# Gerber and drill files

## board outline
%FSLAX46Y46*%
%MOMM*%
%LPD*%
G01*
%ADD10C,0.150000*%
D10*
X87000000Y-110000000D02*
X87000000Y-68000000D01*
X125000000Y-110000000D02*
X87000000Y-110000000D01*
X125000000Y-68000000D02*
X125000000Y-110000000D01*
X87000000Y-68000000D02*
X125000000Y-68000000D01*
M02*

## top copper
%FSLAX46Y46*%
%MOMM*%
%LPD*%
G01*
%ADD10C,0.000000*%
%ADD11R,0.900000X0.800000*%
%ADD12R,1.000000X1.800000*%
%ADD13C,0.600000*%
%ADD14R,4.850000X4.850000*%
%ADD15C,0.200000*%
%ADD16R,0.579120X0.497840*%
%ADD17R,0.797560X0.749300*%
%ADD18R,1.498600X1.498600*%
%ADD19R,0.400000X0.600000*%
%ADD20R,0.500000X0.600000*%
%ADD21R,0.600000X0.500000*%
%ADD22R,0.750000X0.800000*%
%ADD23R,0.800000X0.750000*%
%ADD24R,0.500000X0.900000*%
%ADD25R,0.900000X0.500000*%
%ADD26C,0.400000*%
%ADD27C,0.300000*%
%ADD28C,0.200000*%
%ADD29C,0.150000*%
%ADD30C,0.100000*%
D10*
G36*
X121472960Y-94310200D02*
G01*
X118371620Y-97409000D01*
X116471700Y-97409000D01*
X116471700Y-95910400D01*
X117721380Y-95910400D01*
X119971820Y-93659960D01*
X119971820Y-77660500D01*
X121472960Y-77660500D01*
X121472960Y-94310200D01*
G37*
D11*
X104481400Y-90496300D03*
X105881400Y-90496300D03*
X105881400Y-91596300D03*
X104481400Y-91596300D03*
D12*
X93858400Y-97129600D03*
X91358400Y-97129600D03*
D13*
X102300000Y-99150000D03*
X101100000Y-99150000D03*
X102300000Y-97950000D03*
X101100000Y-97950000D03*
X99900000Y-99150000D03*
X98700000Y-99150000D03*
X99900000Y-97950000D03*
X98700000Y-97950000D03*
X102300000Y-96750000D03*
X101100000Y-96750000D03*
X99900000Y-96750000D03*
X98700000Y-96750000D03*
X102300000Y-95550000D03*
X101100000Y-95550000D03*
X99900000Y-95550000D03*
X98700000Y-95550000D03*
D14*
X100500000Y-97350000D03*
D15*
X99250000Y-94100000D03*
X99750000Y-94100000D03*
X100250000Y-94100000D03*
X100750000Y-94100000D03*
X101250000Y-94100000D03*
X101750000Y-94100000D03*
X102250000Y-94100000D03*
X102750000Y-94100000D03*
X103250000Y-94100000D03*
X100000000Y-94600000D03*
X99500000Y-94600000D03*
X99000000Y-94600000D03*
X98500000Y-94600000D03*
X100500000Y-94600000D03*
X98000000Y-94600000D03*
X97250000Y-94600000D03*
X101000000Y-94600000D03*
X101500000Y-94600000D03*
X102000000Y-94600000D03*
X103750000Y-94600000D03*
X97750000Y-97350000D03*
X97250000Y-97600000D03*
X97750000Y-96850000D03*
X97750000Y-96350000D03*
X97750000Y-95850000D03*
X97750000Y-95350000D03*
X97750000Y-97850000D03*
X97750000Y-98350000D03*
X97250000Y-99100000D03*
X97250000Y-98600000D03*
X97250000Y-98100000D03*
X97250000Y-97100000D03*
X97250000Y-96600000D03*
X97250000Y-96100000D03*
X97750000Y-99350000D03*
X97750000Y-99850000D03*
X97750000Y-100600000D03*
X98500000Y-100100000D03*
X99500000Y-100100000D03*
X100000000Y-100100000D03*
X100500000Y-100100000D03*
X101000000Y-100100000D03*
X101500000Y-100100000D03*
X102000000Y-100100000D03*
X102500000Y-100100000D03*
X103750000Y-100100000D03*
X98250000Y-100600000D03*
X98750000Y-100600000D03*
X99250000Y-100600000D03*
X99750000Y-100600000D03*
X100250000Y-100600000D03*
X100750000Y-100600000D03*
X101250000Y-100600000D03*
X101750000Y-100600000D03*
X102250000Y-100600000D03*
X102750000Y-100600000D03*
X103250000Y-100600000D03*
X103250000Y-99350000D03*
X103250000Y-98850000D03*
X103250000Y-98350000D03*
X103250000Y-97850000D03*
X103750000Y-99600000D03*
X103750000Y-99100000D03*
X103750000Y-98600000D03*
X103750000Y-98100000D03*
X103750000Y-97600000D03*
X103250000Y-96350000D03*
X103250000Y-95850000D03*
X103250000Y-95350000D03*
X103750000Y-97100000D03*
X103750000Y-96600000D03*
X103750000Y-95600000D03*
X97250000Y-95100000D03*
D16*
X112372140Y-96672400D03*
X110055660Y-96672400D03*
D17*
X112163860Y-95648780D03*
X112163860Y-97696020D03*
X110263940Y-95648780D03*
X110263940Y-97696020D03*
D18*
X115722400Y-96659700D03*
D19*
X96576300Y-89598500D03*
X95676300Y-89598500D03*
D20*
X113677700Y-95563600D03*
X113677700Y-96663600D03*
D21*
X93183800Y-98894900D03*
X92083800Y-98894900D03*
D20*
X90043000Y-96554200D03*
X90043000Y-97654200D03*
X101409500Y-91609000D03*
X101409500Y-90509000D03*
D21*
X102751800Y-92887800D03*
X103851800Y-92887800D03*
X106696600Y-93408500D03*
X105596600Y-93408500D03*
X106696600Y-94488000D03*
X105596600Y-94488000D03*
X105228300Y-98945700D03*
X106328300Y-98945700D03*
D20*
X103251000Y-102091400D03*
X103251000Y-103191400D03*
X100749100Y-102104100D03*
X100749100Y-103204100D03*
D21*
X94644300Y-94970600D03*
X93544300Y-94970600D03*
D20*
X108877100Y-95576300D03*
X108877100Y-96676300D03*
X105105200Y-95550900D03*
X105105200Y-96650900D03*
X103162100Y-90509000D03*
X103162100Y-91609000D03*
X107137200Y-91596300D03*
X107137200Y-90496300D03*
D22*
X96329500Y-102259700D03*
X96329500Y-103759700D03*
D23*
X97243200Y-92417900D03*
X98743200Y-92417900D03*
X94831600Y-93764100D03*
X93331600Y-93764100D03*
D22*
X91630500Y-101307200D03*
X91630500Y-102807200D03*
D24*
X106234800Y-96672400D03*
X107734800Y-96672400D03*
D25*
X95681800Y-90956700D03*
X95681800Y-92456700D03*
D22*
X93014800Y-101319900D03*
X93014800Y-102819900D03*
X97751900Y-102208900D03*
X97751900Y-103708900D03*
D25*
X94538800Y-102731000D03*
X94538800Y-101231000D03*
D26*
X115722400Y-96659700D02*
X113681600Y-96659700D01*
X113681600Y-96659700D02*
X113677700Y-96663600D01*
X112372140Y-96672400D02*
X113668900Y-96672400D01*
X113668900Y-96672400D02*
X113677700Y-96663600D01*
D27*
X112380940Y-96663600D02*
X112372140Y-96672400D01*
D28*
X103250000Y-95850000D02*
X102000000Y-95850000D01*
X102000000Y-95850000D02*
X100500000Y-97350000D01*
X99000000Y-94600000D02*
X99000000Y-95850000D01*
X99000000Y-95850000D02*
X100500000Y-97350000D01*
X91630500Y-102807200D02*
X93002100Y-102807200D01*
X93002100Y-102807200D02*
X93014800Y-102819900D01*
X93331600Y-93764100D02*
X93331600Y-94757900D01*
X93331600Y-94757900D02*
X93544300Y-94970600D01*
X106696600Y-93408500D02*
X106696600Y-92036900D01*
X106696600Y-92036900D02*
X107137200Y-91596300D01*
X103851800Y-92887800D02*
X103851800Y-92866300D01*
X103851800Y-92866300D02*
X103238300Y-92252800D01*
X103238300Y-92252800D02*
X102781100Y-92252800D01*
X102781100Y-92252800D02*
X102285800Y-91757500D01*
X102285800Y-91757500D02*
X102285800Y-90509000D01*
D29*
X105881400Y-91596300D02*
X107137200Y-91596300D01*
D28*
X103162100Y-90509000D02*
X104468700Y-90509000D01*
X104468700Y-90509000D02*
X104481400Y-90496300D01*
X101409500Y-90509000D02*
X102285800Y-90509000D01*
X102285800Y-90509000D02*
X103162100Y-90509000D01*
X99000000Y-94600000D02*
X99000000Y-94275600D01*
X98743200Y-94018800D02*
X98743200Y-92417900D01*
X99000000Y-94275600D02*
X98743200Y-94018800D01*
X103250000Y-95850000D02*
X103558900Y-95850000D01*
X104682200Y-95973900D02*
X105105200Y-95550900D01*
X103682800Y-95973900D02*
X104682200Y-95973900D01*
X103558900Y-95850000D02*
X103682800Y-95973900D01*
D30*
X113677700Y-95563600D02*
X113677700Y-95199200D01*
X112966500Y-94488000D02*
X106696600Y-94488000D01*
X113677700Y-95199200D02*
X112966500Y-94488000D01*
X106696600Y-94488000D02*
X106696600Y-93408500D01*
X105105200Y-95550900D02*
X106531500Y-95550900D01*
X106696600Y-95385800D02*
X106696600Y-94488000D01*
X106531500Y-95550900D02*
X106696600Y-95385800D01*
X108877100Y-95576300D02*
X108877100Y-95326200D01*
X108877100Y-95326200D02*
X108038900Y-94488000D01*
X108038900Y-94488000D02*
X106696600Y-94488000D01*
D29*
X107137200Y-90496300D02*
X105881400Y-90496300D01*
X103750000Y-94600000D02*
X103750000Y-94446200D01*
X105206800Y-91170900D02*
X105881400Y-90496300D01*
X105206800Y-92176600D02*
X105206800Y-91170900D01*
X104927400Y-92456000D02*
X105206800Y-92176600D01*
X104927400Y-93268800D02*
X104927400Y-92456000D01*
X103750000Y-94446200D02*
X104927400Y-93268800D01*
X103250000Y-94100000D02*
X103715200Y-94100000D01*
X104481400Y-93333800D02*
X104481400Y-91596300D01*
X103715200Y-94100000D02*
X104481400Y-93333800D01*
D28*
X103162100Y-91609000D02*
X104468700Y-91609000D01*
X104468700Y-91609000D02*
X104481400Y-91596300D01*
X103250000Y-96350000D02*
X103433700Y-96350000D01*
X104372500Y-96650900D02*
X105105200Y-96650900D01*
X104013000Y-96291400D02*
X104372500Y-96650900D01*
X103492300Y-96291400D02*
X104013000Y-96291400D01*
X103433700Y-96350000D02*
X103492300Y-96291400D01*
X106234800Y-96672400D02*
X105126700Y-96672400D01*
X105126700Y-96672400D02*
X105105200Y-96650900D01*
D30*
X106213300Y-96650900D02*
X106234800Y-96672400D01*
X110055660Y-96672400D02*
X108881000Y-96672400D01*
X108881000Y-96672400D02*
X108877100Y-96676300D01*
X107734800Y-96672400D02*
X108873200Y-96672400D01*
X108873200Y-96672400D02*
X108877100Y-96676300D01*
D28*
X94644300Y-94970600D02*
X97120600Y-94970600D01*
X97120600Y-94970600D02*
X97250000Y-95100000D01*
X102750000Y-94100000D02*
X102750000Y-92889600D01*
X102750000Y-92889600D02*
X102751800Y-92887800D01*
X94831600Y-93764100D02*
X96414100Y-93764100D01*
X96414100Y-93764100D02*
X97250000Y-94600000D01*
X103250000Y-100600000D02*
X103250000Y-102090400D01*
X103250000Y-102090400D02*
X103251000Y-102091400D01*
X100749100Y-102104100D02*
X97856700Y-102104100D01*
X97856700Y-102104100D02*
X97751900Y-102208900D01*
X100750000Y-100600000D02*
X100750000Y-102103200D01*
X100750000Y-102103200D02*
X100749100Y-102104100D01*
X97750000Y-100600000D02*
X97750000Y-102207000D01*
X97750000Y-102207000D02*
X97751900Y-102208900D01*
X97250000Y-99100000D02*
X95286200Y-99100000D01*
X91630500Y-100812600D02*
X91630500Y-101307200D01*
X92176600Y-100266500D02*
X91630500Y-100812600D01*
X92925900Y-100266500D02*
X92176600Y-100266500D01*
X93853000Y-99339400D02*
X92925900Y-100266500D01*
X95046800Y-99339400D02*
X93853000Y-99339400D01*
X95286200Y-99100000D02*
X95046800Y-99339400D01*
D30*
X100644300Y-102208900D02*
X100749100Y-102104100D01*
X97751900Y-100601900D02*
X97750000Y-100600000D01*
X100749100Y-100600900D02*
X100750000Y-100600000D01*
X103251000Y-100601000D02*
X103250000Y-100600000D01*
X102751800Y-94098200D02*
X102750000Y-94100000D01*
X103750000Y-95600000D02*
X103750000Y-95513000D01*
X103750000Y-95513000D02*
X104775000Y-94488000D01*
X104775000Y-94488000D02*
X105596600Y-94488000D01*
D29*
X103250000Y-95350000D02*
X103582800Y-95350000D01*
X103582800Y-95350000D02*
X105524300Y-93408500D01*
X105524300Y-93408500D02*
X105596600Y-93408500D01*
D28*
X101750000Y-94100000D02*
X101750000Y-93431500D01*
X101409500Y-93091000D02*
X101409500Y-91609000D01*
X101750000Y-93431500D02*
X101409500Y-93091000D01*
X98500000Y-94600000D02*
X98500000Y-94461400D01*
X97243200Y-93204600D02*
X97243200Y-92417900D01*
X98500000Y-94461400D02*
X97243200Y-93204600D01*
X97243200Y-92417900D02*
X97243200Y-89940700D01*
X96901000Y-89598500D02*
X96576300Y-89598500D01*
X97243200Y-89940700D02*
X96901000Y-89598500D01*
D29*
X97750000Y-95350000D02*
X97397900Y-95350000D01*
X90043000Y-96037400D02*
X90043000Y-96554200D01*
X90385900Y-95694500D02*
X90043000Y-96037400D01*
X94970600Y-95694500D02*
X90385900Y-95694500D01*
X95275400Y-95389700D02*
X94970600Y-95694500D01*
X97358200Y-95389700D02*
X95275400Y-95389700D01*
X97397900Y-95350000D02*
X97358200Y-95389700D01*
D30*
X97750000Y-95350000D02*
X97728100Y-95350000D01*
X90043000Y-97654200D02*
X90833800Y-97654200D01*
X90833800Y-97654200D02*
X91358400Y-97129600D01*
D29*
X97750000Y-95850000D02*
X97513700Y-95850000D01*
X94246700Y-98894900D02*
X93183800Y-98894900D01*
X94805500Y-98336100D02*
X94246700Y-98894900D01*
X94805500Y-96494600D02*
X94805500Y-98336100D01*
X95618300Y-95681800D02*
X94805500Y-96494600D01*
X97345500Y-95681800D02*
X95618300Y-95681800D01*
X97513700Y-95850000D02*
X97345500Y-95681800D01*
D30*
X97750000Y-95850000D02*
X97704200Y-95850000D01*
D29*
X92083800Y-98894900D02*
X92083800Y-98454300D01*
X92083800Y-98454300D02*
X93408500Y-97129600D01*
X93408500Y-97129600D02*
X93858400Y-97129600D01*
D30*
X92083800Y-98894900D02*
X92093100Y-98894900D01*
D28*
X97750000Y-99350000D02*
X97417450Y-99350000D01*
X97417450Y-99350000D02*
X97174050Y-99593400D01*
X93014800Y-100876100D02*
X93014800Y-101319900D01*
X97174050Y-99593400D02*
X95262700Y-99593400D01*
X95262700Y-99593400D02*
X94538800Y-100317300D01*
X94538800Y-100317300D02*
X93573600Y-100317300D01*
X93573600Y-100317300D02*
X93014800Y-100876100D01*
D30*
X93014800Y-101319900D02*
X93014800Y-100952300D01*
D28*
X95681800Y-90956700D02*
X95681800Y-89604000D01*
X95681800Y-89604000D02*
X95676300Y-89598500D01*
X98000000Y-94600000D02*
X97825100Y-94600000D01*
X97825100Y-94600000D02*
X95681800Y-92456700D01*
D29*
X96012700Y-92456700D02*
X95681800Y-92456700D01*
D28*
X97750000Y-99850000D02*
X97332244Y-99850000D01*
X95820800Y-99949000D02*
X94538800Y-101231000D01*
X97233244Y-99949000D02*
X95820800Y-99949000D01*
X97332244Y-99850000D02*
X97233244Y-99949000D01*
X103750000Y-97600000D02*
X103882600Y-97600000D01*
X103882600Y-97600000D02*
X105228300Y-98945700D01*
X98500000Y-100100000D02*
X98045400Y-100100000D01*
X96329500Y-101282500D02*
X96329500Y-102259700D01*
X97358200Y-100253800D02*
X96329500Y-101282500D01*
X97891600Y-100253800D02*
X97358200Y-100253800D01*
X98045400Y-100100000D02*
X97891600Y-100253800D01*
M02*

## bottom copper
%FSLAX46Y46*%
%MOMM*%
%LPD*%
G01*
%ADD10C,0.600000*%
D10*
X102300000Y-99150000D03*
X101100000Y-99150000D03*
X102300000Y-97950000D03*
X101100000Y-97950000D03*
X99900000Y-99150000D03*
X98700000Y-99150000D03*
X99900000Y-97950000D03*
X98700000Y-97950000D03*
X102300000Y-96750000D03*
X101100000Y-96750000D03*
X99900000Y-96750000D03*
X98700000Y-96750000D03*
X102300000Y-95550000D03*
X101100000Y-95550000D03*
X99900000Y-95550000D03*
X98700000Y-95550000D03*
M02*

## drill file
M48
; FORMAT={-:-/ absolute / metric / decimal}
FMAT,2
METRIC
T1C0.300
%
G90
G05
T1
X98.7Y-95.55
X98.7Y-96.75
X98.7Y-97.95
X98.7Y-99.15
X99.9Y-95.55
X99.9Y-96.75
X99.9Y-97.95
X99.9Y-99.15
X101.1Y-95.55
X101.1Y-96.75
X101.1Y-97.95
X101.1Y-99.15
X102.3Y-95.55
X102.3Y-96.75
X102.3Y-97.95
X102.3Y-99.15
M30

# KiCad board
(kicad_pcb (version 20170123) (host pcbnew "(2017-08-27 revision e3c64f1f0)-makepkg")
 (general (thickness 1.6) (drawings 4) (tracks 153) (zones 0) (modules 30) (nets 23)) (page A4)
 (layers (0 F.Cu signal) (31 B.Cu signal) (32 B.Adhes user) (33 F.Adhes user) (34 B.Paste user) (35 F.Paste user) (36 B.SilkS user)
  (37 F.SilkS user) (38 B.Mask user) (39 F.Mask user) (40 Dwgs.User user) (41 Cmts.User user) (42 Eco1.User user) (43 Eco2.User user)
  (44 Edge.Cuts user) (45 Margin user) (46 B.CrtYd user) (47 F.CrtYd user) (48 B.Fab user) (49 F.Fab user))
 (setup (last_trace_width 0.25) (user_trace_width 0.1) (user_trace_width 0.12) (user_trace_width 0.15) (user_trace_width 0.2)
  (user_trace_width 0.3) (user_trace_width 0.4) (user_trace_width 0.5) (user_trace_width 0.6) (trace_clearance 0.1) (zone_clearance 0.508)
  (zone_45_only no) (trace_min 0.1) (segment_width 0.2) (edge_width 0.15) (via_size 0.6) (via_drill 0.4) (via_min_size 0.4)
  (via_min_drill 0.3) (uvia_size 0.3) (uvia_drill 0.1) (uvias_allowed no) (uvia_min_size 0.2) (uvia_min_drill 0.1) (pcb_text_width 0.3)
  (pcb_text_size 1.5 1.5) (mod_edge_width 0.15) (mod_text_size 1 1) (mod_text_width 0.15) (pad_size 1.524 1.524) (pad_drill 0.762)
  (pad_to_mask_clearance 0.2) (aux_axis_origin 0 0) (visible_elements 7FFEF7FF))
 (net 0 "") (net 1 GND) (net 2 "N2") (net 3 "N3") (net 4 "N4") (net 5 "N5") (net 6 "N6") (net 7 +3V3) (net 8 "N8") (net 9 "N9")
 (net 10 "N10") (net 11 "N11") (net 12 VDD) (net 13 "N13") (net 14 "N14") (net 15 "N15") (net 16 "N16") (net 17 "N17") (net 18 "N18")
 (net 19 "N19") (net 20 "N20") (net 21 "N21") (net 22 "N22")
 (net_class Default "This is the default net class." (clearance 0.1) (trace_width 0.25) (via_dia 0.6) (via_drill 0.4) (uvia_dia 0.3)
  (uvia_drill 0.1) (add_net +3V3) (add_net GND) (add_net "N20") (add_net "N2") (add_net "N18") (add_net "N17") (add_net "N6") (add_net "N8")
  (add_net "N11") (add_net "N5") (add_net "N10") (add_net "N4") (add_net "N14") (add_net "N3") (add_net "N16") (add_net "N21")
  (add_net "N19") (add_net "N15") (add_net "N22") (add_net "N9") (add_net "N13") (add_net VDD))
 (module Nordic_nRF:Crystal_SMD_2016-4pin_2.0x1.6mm (layer F.Cu) (at 105.1814 91.0463)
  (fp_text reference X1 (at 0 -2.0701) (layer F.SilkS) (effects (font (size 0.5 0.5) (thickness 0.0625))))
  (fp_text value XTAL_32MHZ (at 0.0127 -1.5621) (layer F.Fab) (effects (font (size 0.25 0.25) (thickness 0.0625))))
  (pad 4 smd rect (at -0.7 -0.55) (size 0.9 0.8) (layers F.Cu F.Paste F.Mask) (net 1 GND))
  (pad 3 smd rect (at 0.7 -0.55) (size 0.9 0.8) (layers F.Cu F.Paste F.Mask) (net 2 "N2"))
  (pad 2 smd rect (at 0.7 0.55) (size 0.9 0.8) (layers F.Cu F.Paste F.Mask) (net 1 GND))
  (pad 1 smd rect (at -0.7 0.55) (size 0.9 0.8) (layers F.Cu F.Paste F.Mask) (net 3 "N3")))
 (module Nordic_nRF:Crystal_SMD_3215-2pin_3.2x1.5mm (layer F.Cu) (at 92.6084 97.1296 180)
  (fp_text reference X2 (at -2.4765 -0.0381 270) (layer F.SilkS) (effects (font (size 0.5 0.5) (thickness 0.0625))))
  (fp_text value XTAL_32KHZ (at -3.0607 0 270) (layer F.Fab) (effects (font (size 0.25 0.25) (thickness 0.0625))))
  (pad 2 smd rect (at -1.25 0 180) (size 1 1.8) (layers F.Cu F.Paste F.Mask) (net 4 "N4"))
  (pad 1 smd rect (at 1.25 0 180) (size 1 1.8) (layers F.Cu F.Paste F.Mask) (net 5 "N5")))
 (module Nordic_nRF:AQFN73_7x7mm (layer F.Cu) (at 100.5 97.35)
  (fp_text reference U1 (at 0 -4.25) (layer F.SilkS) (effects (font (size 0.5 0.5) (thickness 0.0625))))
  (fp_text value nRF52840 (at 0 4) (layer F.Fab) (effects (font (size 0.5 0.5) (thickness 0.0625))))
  (pad 74 thru_hole circle (at 1.8 1.8) (size 0.6 0.6) (drill 0.3) (layers *.Cu B.Mask) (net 1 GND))
  (pad 74 thru_hole circle (at 0.6 1.8) (size 0.6 0.6) (drill 0.3) (layers *.Cu B.Mask) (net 1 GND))
  (pad 74 thru_hole circle (at 1.8 0.6) (size 0.6 0.6) (drill 0.3) (layers *.Cu B.Mask) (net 1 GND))
  (pad 74 thru_hole circle (at 0.6 0.6) (size 0.6 0.6) (drill 0.3) (layers *.Cu B.Mask) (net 1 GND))
  (pad 74 thru_hole circle (at -0.6 1.8) (size 0.6 0.6) (drill 0.3) (layers *.Cu B.Mask) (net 1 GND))
  (pad 74 thru_hole circle (at -1.8 1.8) (size 0.6 0.6) (drill 0.3) (layers *.Cu B.Mask) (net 1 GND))
  (pad 74 thru_hole circle (at -0.6 0.6) (size 0.6 0.6) (drill 0.3) (layers *.Cu B.Mask) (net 1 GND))
  (pad 74 thru_hole circle (at -1.8 0.6) (size 0.6 0.6) (drill 0.3) (layers *.Cu B.Mask) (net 1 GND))
  (pad 74 thru_hole circle (at 1.8 -0.6) (size 0.6 0.6) (drill 0.3) (layers *.Cu B.Mask) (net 1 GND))
  (pad 74 thru_hole circle (at 0.6 -0.6) (size 0.6 0.6) (drill 0.3) (layers *.Cu B.Mask) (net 1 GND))
  (pad 74 thru_hole circle (at -0.6 -0.6) (size 0.6 0.6) (drill 0.3) (layers *.Cu B.Mask) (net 1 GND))
  (pad 74 thru_hole circle (at -1.8 -0.6) (size 0.6 0.6) (drill 0.3) (layers *.Cu B.Mask) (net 1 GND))
  (pad 74 thru_hole circle (at 1.8 -1.8) (size 0.6 0.6) (drill 0.3) (layers *.Cu B.Mask) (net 1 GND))
  (pad 74 thru_hole circle (at 0.6 -1.8) (size 0.6 0.6) (drill 0.3) (layers *.Cu B.Mask) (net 1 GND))
  (pad 74 thru_hole circle (at -0.6 -1.8) (size 0.6 0.6) (drill 0.3) (layers *.Cu B.Mask) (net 1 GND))
  (pad 74 thru_hole circle (at -1.8 -1.8) (size 0.6 0.6) (drill 0.3) (layers *.Cu B.Mask) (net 1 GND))
  (pad 74 smd rect (at 0 0) (size 4.85 4.85) (layers F.Cu F.Paste F.Mask) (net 1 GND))
  (pad A8 smd circle (at -1.25 -3.25) (size 0.2 0.2) (layers F.Cu F.Paste F.Mask))
  (pad A10 smd circle (at -0.75 -3.25) (size 0.2 0.2) (layers F.Cu F.Paste F.Mask))
  (pad A12 smd circle (at -0.25 -3.25) (size 0.2 0.2) (layers F.Cu F.Paste F.Mask))
  (pad A14 smd circle (at 0.25 -3.25) (size 0.2 0.2) (layers F.Cu F.Paste F.Mask))
  (pad A16 smd circle (at 0.75 -3.25) (size 0.2 0.2) (layers F.Cu F.Paste F.Mask))
  (pad A18 smd circle (at 1.25 -3.25) (size 0.2 0.2) (layers F.Cu F.Paste F.Mask) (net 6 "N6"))
  (pad A20 smd circle (at 1.75 -3.25) (size 0.2 0.2) (layers F.Cu F.Paste F.Mask))
  (pad A22 smd circle (at 2.25 -3.25) (size 0.2 0.2) (layers F.Cu F.Paste F.Mask) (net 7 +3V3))
  (pad A23 smd circle (at 2.75 -3.25) (size 0.2 0.2) (layers F.Cu F.Paste F.Mask) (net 3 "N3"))
  (pad B11 smd circle (at -0.5 -2.75) (size 0.2 0.2) (layers F.Cu F.Paste F.Mask))
  (pad B9 smd circle (at -1 -2.75) (size 0.2 0.2) (layers F.Cu F.Paste F.Mask))
  (pad B7 smd circle (at -1.5 -2.75) (size 0.2 0.2) (layers F.Cu F.Paste F.Mask) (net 1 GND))
  (pad B5 smd circle (at -2 -2.75) (size 0.2 0.2) (layers F.Cu F.Paste F.Mask) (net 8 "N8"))
  (pad B13 smd circle (at 0 -2.75) (size 0.2 0.2) (layers F.Cu F.Paste F.Mask))
  (pad B3 smd circle (at -2.5 -2.75) (size 0.2 0.2) (layers F.Cu F.Paste F.Mask) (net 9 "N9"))
  (pad B1 smd circle (at -3.25 -2.75) (size 0.2 0.2) (layers F.Cu F.Paste F.Mask) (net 7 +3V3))
  (pad B15 smd circle (at 0.5 -2.75) (size 0.2 0.2) (layers F.Cu F.Paste F.Mask))
  (pad B17 smd circle (at 1 -2.75) (size 0.2 0.2) (layers F.Cu F.Paste F.Mask))
  (pad B19 smd circle (at 1.5 -2.75) (size 0.2 0.2) (layers F.Cu F.Paste F.Mask))
  (pad B24 smd circle (at 3.25 -2.75) (size 0.2 0.2) (layers F.Cu F.Paste F.Mask) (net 2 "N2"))
  (pad M2 smd circle (at -2.75 0) (size 0.2 0.2) (layers F.Cu F.Paste F.Mask))
  (pad N1 smd circle (at -3.25 0.25) (size 0.2 0.2) (layers F.Cu F.Paste F.Mask))
  (pad K2 smd circle (at -2.75 -0.5) (size 0.2 0.2) (layers F.Cu F.Paste F.Mask))
  (pad H2 smd circle (at -2.75 -1) (size 0.2 0.2) (layers F.Cu F.Paste F.Mask))
  (pad F2 smd circle (at -2.75 -1.5) (size 0.2 0.2) (layers F.Cu F.Paste F.Mask) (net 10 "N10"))
  (pad D2 smd circle (at -2.75 -2) (size 0.2 0.2) (layers F.Cu F.Paste F.Mask) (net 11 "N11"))
  (pad P2 smd circle (at -2.75 0.5) (size 0.2 0.2) (layers F.Cu F.Paste F.Mask))
  (pad T2 smd circle (at -2.75 1) (size 0.2 0.2) (layers F.Cu F.Paste F.Mask))
  (pad W1 smd circle (at -3.25 1.75) (size 0.2 0.2) (layers F.Cu F.Paste F.Mask) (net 7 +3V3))
  (pad U1 smd circle (at -3.25 1.25) (size 0.2 0.2) (layers F.Cu F.Paste F.Mask))
  (pad R1 smd circle (at -3.25 0.75) (size 0.2 0.2) (layers F.Cu F.Paste F.Mask))
  (pad L1 smd circle (at -3.25 -0.25) (size 0.2 0.2) (layers F.Cu F.Paste F.Mask))
  (pad J1 smd circle (at -3.25 -0.75) (size 0.2 0.2) (layers F.Cu F.Paste F.Mask))
  (pad G1 smd circle (at -3.25 -1.25) (size 0.2 0.2) (layers F.Cu F.Paste F.Mask))
  (pad Y2 smd circle (at -2.75 2) (size 0.2 0.2) (layers F.Cu F.Paste F.Mask) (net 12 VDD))
  (pad AB2 smd circle (at -2.75 2.5) (size 0.2 0.2) (layers F.Cu F.Paste F.Mask) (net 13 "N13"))
  (pad AD2 smd circle (at -2.75 3.25) (size 0.2 0.2) (layers F.Cu F.Paste F.Mask) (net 7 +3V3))
  (pad AC5 smd circle (at -2 2.75) (size 0.2 0.2) (layers F.Cu F.Paste F.Mask) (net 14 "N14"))
  (pad AC9 smd circle (at -1 2.75) (size 0.2 0.2) (layers F.Cu F.Paste F.Mask))
  (pad AC11 smd circle (at -0.5 2.75) (size 0.2 0.2) (layers F.Cu F.Paste F.Mask))
  (pad AC13 smd circle (at 0 2.75) (size 0.2 0.2) (layers F.Cu F.Paste F.Mask))
  (pad AC15 smd circle (at 0.5 2.75) (size 0.2 0.2) (layers F.Cu F.Paste F.Mask))
  (pad AC17 smd circle (at 1 2.75) (size 0.2 0.2) (layers F.Cu F.Paste F.Mask))
  (pad AC19 smd circle (at 1.5 2.75) (size 0.2 0.2) (layers F.Cu F.Paste F.Mask))
  (pad AC21 smd circle (at 2 2.75) (size 0.2 0.2) (layers F.Cu F.Paste F.Mask))
  (pad AC24 smd circle (at 3.25 2.75) (size 0.2 0.2) (layers F.Cu F.Paste F.Mask))
  (pad AD4 smd circle (at -2.25 3.25) (size 0.2 0.2) (layers F.Cu F.Paste F.Mask))
  (pad AD6 smd circle (at -1.75 3.25) (size 0.2 0.2) (layers F.Cu F.Paste F.Mask))
  (pad AD8 smd circle (at -1.25 3.25) (size 0.2 0.2) (layers F.Cu F.Paste F.Mask))
  (pad AD10 smd circle (at -0.75 3.25) (size 0.2 0.2) (layers F.Cu F.Paste F.Mask))
  (pad AD12 smd circle (at -0.25 3.25) (size 0.2 0.2) (layers F.Cu F.Paste F.Mask))
  (pad AD14 smd circle (at 0.25 3.25) (size 0.2 0.2) (layers F.Cu F.Paste F.Mask) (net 7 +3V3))
  (pad AD16 smd circle (at 0.75 3.25) (size 0.2 0.2) (layers F.Cu F.Paste F.Mask))
  (pad AD18 smd circle (at 1.25 3.25) (size 0.2 0.2) (layers F.Cu F.Paste F.Mask))
  (pad AD20 smd circle (at 1.75 3.25) (size 0.2 0.2) (layers F.Cu F.Paste F.Mask))
  (pad AD22 smd circle (at 2.25 3.25) (size 0.2 0.2) (layers F.Cu F.Paste F.Mask))
  (pad AD23 smd circle (at 2.75 3.25) (size 0.2 0.2) (layers F.Cu F.Paste F.Mask) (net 7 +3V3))
  (pad Y23 smd circle (at 2.75 2) (size 0.2 0.2) (layers F.Cu F.Paste F.Mask))
  (pad V23 smd circle (at 2.75 1.5) (size 0.2 0.2) (layers F.Cu F.Paste F.Mask))
  (pad T23 smd circle (at 2.75 1) (size 0.2 0.2) (layers F.Cu F.Paste F.Mask))
  (pad P23 smd circle (at 2.75 0.5) (size 0.2 0.2) (layers F.Cu F.Paste F.Mask))
  (pad AA24 smd circle (at 3.25 2.25) (size 0.2 0.2) (layers F.Cu F.Paste F.Mask))
  (pad W24 smd circle (at 3.25 1.75) (size 0.2 0.2) (layers F.Cu F.Paste F.Mask))
  (pad U24 smd circle (at 3.25 1.25) (size 0.2 0.2) (layers F.Cu F.Paste F.Mask))
  (pad R24 smd circle (at 3.25 0.75) (size 0.2 0.2) (layers F.Cu F.Paste F.Mask))
  (pad N24 smd circle (at 3.25 0.25) (size 0.2 0.2) (layers F.Cu F.Paste F.Mask) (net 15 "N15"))
  (pad H23 smd circle (at 2.75 -1) (size 0.2 0.2) (layers F.Cu F.Paste F.Mask) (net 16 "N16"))
  (pad F23 smd circle (at 2.75 -1.5) (size 0.2 0.2) (layers F.Cu F.Paste F.Mask) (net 1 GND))
  (pad D23 smd circle (at 2.75 -2) (size 0.2 0.2) (layers F.Cu F.Paste F.Mask) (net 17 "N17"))
  (pad L24 smd circle (at 3.25 -0.25) (size 0.2 0.2) (layers F.Cu F.Paste F.Mask))
  (pad J24 smd circle (at 3.25 -0.75) (size 0.2 0.2) (layers F.Cu F.Paste F.Mask))
  (pad E24 smd circle (at 3.25 -1.75) (size 0.2 0.2) (layers F.Cu F.Paste F.Mask) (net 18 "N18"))
  (pad C1 smd circle (at -3.25 -2.25) (size 0.2 0.2) (layers F.Cu F.Paste F.Mask) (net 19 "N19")))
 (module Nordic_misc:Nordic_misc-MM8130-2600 (layer F.Cu) (at 111.2139 96.6724 90)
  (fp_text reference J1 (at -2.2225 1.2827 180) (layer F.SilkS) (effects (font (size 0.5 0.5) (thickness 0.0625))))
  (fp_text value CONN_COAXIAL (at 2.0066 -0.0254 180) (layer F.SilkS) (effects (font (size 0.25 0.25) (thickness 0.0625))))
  (pad 2 smd rect (at 0 1.15824 90) (size 0.49784 0.57912) (layers F.Cu F.Paste F.Mask) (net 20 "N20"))
  (pad 1 smd rect (at 0 -1.15824 90) (size 0.49784 0.57912) (layers F.Cu F.Paste F.Mask) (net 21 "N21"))
  (pad 0 smd rect (at 1.02362 0.94996 90) (size 0.7493 0.79756) (layers F.Cu F.Paste F.Mask))
  (pad 0 smd rect (at -1.02362 0.94996 90) (size 0.7493 0.79756) (layers F.Cu F.Paste F.Mask))
  (pad 0 smd rect (at 1.02362 -0.94996 90) (size 0.7493 0.79756) (layers F.Cu F.Paste F.Mask))
  (pad 0 smd rect (at -1.02362 -0.94996 90) (size 0.7493 0.79756) (layers F.Cu F.Paste F.Mask)))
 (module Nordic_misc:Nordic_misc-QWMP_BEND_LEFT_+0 (layer F.Cu) (at 114.9731 96.6597)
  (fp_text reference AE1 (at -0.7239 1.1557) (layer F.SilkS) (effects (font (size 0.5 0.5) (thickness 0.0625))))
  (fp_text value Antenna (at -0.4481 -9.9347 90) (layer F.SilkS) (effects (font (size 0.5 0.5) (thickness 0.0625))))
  (fp_poly
   (pts (xy 1.4986 -0.7493) (xy 2.74828 -0.7493) (xy 4.99872 -2.99974) (xy 4.99872 -18.9992) (xy 6.49986 -18.9992) (xy 6.49986 -2.3495)
    (xy 3.39852 0.7493) (xy 1.4986 0.7493) (xy 1.4986 -0.7493))
   (layer F.Cu) (width 0))
  (pad 1 smd rect (at 0.7493 0) (size 1.4986 1.4986) (layers F.Cu F.Paste F.Mask) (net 20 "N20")))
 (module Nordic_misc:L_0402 (layer F.Cu) (at 96.1263 89.5985 180)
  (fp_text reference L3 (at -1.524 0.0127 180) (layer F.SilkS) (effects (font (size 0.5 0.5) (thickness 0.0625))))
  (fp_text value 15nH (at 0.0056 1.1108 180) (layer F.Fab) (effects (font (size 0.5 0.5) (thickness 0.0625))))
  (pad 1 smd rect (at -0.45 0 180) (size 0.4 0.6) (layers F.Cu F.Paste F.Mask) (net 8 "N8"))
  (pad 2 smd rect (at 0.45 0 180) (size 0.4 0.6) (layers F.Cu F.Paste F.Mask) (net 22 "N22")))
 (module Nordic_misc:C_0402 (layer F.Cu) (at 113.6777 96.1136 270)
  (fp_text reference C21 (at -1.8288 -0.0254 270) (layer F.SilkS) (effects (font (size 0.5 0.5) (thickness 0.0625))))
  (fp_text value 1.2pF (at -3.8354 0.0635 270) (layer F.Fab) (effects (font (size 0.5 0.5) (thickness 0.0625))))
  (pad 1 smd rect (at -0.55 0 270) (size 0.6 0.5) (layers F.Cu F.Paste F.Mask) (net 1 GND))
  (pad 2 smd rect (at 0.55 0 270) (size 0.6 0.5) (layers F.Cu F.Paste F.Mask) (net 20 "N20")))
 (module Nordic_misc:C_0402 (layer F.Cu) (at 92.6338 98.8949 180)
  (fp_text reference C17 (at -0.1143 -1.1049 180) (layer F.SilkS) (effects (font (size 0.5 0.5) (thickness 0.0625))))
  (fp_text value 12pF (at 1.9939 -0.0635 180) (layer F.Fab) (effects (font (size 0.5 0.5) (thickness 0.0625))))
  (pad 1 smd rect (at -0.55 0 180) (size 0.6 0.5) (layers F.Cu F.Paste F.Mask) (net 10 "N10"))
  (pad 2 smd rect (at 0.55 0 180) (size 0.6 0.5) (layers F.Cu F.Paste F.Mask) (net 4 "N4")))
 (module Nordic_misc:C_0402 (layer F.Cu) (at 90.043 97.1042 270)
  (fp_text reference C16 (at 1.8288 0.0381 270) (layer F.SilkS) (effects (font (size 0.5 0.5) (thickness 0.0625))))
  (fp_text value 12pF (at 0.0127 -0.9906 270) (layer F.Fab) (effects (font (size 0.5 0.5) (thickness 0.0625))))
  (pad 1 smd rect (at -0.55 0 270) (size 0.6 0.5) (layers F.Cu F.Paste F.Mask) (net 11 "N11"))
  (pad 2 smd rect (at 0.55 0 270) (size 0.6 0.5) (layers F.Cu F.Paste F.Mask) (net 5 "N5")))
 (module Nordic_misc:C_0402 (layer F.Cu) (at 101.4095 91.059 90)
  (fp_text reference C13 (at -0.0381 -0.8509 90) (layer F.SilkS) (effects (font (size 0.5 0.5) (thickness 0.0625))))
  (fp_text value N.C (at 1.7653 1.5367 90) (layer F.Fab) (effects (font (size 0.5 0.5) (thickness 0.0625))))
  (pad 1 smd rect (at -0.55 0 90) (size 0.6 0.5) (layers F.Cu F.Paste F.Mask) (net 6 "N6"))
  (pad 2 smd rect (at 0.55 0 90) (size 0.6 0.5) (layers F.Cu F.Paste F.Mask) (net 1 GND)))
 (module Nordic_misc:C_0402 (layer F.Cu) (at 103.3018 92.8878)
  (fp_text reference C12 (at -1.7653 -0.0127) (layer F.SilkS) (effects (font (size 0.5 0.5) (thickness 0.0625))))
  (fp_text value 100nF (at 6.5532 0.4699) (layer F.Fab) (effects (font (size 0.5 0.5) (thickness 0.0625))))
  (pad 1 smd rect (at -0.55 0) (size 0.6 0.5) (layers F.Cu F.Paste F.Mask) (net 7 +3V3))
  (pad 2 smd rect (at 0.55 0) (size 0.6 0.5) (layers F.Cu F.Paste F.Mask) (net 1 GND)))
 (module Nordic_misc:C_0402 (layer F.Cu) (at 106.1466 93.4085 180)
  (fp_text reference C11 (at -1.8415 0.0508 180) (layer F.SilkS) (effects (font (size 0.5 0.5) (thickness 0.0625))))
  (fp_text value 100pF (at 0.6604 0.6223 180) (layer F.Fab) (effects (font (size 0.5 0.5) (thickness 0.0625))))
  (pad 1 smd rect (at -0.55 0 180) (size 0.6 0.5) (layers F.Cu F.Paste F.Mask) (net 1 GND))
  (pad 2 smd rect (at 0.55 0 180) (size 0.6 0.5) (layers F.Cu F.Paste F.Mask) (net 17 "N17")))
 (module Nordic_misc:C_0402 (layer F.Cu) (at 106.1466 94.488 180)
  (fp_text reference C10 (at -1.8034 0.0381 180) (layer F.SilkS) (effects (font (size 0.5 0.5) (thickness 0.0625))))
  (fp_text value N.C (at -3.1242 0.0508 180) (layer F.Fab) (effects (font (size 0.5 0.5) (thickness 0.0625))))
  (pad 1 smd rect (at -0.55 0 180) (size 0.6 0.5) (layers F.Cu F.Paste F.Mask) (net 1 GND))
  (pad 2 smd rect (at 0.55 0 180) (size 0.6 0.5) (layers F.Cu F.Paste F.Mask) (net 18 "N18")))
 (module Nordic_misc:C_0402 (layer F.Cu) (at 105.7783 98.9457)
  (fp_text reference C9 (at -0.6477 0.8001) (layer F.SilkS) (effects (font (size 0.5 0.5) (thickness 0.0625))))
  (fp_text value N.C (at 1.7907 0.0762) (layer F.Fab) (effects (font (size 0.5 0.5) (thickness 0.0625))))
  (pad 1 smd rect (at -0.55 0) (size 0.6 0.5) (layers F.Cu F.Paste F.Mask) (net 15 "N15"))
  (pad 2 smd rect (at 0.55 0) (size 0.6 0.5) (layers F.Cu F.Paste F.Mask) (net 1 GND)))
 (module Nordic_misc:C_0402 (layer F.Cu) (at 103.251 102.6414 270)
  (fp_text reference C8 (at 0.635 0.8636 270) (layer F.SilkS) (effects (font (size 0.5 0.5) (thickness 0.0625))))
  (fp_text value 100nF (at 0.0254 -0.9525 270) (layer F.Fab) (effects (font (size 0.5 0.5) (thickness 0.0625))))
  (pad 1 smd rect (at -0.55 0 270) (size 0.6 0.5) (layers F.Cu F.Paste F.Mask) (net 7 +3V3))
  (pad 2 smd rect (at 0.55 0 270) (size 0.6 0.5) (layers F.Cu F.Paste F.Mask) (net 1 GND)))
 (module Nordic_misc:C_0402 (layer F.Cu) (at 100.7491 102.6541 270)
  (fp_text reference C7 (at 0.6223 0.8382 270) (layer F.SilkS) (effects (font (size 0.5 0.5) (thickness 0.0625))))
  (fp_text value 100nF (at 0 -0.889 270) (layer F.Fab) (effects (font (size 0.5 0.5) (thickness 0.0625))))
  (pad 1 smd rect (at -0.55 0 270) (size 0.6 0.5) (layers F.Cu F.Paste F.Mask) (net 7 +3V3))
  (pad 2 smd rect (at 0.55 0 270) (size 0.6 0.5) (layers F.Cu F.Paste F.Mask) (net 1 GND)))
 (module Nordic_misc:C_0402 (layer F.Cu) (at 94.0943 94.9706 180)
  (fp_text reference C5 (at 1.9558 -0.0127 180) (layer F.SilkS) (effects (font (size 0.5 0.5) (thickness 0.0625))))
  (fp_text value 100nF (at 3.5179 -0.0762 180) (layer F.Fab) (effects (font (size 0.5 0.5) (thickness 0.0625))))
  (pad 1 smd rect (at -0.55 0 180) (size 0.6 0.5) (layers F.Cu F.Paste F.Mask) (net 19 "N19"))
  (pad 2 smd rect (at 0.55 0 180) (size 0.6 0.5) (layers F.Cu F.Paste F.Mask) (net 1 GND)))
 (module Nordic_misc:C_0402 (layer F.Cu) (at 108.8771 96.1263 270)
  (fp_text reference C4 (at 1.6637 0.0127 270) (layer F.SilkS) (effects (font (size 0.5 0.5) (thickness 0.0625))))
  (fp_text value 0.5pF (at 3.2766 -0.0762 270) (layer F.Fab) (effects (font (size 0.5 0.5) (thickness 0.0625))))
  (pad 1 smd rect (at -0.55 0 270) (size 0.6 0.5) (layers F.Cu F.Paste F.Mask) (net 1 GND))
  (pad 2 smd rect (at 0.55 0 270) (size 0.6 0.5) (layers F.Cu F.Paste F.Mask) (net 21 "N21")))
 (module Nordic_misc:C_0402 (layer F.Cu) (at 105.1052 96.1009 270)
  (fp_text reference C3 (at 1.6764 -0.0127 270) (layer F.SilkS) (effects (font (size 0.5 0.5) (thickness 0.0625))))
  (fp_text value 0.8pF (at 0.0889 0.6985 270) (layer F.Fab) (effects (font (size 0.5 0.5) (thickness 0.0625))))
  (pad 1 smd rect (at -0.55 0 270) (size 0.6 0.5) (layers F.Cu F.Paste F.Mask) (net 1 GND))
  (pad 2 smd rect (at 0.55 0 270) (size 0.6 0.5) (layers F.Cu F.Paste F.Mask) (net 16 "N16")))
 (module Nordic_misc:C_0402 (layer F.Cu) (at 103.1621 91.059 270)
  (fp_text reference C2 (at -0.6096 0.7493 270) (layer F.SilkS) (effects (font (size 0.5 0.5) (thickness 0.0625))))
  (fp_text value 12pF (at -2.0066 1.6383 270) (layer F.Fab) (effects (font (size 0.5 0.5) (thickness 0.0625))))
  (pad 1 smd rect (at -0.55 0 270) (size 0.6 0.5) (layers F.Cu F.Paste F.Mask) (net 1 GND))
  (pad 2 smd rect (at 0.55 0 270) (size 0.6 0.5) (layers F.Cu F.Paste F.Mask) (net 3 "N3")))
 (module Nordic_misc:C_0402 (layer F.Cu) (at 107.1372 91.0463 90)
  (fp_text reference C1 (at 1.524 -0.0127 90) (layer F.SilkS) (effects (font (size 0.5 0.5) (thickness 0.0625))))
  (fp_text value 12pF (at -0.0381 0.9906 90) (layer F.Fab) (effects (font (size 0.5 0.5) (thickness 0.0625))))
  (pad 1 smd rect (at -0.55 0 90) (size 0.6 0.5) (layers F.Cu F.Paste F.Mask) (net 1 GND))
  (pad 2 smd rect (at 0.55 0 90) (size 0.6 0.5) (layers F.Cu F.Paste F.Mask) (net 2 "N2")))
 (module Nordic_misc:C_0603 (layer F.Cu) (at 96.3295 103.0097 270)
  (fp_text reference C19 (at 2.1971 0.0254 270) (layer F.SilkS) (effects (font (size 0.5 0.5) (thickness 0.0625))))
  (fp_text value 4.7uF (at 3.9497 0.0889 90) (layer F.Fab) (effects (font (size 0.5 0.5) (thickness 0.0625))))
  (pad 1 smd rect (at -0.75 0 270) (size 0.8 0.75) (layers F.Cu F.Paste F.Mask) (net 14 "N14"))
  (pad 2 smd rect (at 0.75 0 270) (size 0.8 0.75) (layers F.Cu F.Paste F.Mask) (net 1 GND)))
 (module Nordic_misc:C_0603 (layer F.Cu) (at 97.9932 92.4179)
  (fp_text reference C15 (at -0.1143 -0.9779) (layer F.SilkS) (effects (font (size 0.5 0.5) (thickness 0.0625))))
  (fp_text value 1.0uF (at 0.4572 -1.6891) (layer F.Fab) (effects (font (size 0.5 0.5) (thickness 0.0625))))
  (pad 1 smd rect (at -0.75 0) (size 0.8 0.75) (layers F.Cu F.Paste F.Mask) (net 8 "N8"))
  (pad 2 smd rect (at 0.75 0) (size 0.8 0.75) (layers F.Cu F.Paste F.Mask) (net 1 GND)))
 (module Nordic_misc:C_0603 (layer F.Cu) (at 94.0816 93.7641 180)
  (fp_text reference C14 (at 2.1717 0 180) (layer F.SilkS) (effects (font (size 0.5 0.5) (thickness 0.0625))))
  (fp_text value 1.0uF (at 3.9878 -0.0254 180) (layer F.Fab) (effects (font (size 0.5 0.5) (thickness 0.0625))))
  (pad 1 smd rect (at -0.75 0 180) (size 0.8 0.75) (layers F.Cu F.Paste F.Mask) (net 7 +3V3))
  (pad 2 smd rect (at 0.75 0 180) (size 0.8 0.75) (layers F.Cu F.Paste F.Mask) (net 1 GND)))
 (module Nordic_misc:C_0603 (layer F.Cu) (at 91.6305 102.0572 270)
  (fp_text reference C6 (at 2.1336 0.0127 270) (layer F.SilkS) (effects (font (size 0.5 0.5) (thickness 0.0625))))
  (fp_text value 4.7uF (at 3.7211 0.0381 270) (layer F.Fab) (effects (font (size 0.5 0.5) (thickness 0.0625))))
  (pad 1 smd rect (at -0.75 0 270) (size 0.8 0.75) (layers F.Cu F.Paste F.Mask) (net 7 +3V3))
  (pad 2 smd rect (at 0.75 0 270) (size 0.8 0.75) (layers F.Cu F.Paste F.Mask) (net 1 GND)))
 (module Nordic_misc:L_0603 (layer F.Cu) (at 106.9848 96.6724)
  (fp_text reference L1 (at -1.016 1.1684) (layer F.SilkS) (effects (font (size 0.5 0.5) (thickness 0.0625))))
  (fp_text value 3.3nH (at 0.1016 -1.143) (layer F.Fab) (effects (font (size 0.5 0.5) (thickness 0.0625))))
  (pad 1 smd rect (at -0.75 0) (size 0.5 0.9) (layers F.Cu F.Paste F.Mask) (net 16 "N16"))
  (pad 2 smd rect (at 0.75 0) (size 0.5 0.9) (layers F.Cu F.Paste F.Mask) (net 21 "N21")))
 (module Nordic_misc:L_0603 (layer F.Cu) (at 95.6818 91.7067 270)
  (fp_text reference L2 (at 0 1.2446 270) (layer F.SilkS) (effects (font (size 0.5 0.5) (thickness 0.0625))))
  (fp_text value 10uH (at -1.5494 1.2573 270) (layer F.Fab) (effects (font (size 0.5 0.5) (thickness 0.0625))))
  (pad 1 smd rect (at -0.75 0 270) (size 0.5 0.9) (layers F.Cu F.Paste F.Mask) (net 22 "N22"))
  (pad 2 smd rect (at 0.75 0 270) (size 0.5 0.9) (layers F.Cu F.Paste F.Mask) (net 9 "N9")))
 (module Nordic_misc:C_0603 (layer F.Cu) (at 93.0148 102.0699 270)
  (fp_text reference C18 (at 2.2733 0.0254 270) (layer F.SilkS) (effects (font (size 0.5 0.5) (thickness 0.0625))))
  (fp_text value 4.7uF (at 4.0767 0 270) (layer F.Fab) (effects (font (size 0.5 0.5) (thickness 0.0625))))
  (pad 1 smd rect (at -0.75 0 270) (size 0.8 0.75) (layers F.Cu F.Paste F.Mask) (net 12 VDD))
  (pad 2 smd rect (at 0.75 0 270) (size 0.8 0.75) (layers F.Cu F.Paste F.Mask) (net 1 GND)))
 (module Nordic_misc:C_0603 (layer F.Cu) (at 97.7519 102.9589 270)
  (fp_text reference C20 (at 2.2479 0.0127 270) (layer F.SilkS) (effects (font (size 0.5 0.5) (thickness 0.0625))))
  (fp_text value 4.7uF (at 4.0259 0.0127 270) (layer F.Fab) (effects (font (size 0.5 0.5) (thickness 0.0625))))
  (pad 1 smd rect (at -0.75 0 270) (size 0.8 0.75) (layers F.Cu F.Paste F.Mask) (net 7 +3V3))
  (pad 2 smd rect (at 0.75 0 270) (size 0.8 0.75) (layers F.Cu F.Paste F.Mask) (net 1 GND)))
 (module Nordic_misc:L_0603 (layer F.Cu) (at 94.5388 101.981 90)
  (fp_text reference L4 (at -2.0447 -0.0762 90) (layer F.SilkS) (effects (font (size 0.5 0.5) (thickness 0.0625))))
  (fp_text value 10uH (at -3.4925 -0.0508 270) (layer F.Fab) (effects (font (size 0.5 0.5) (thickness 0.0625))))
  (pad 1 smd rect (at -0.75 0 90) (size 0.5 0.9) (layers F.Cu F.Paste F.Mask) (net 7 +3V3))
  (pad 2 smd rect (at 0.75 0 90) (size 0.5 0.9) (layers F.Cu F.Paste F.Mask) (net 13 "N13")))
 (gr_line (start 87 110) (end 87 68) (angle 90) (layer Edge.Cuts) (width 0.15))
 (gr_line (start 125 110) (end 87 110) (angle 90) (layer Edge.Cuts) (width 0.15))
 (gr_line (start 125 68) (end 125 110) (angle 90) (layer Edge.Cuts) (width 0.15))
 (gr_line (start 87 68) (end 125 68) (angle 90) (layer Edge.Cuts) (width 0.15))
 (segment (start 115.7224 96.6597) (end 113.6816 96.6597) (width 0.4) (layer F.Cu) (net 20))
 (segment (start 113.6816 96.6597) (end 113.6777 96.6636) (width 0.4) (layer F.Cu) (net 20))
 (segment (start 112.37214 96.6724) (end 113.6689 96.6724) (width 0.4) (layer F.Cu) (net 20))
 (segment (start 113.6689 96.6724) (end 113.6777 96.6636) (width 0.4) (layer F.Cu) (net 20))
 (segment (start 112.38094 96.6636) (end 112.37214 96.6724) (width 0.3) (layer F.Cu) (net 20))
 (segment (start 103.25 95.85) (end 102 95.85) (width 0.2) (layer F.Cu) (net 1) (status C00000))
 (segment (start 102 95.85) (end 100.5 97.35) (width 0.2) (layer F.Cu) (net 1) (status C00000))
 (segment (start 99 94.6) (end 99 95.85) (width 0.2) (layer F.Cu) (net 1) (status C00000))
 (segment (start 99 95.85) (end 100.5 97.35) (width 0.2) (layer F.Cu) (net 1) (status C00000))
 (segment (start 91.6305 102.8072) (end 93.0021 102.8072) (width 0.2) (layer F.Cu) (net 1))
 (segment (start 93.0021 102.8072) (end 93.0148 102.8199) (width 0.2) (layer F.Cu) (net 1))
 (segment (start 93.3316 93.7641) (end 93.3316 94.7579) (width 0.2) (layer F.Cu) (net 1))
 (segment (start 93.3316 94.7579) (end 93.5443 94.9706) (width 0.2) (layer F.Cu) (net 1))
 (segment (start 106.6966 93.4085) (end 106.6966 92.0369) (width 0.2) (layer F.Cu) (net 1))
 (segment (start 106.6966 92.0369) (end 107.1372 91.5963) (width 0.2) (layer F.Cu) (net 1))
 (segment (start 103.8518 92.8878) (end 103.8518 92.8663) (width 0.2) (layer F.Cu) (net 1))
 (segment (start 103.8518 92.8663) (end 103.2383 92.2528) (width 0.2) (layer F.Cu) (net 1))
 (segment (start 103.2383 92.2528) (end 102.7811 92.2528) (width 0.2) (layer F.Cu) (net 1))
 (segment (start 102.7811 92.2528) (end 102.2858 91.7575) (width 0.2) (layer F.Cu) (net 1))
 (segment (start 102.2858 91.7575) (end 102.2858 90.509) (width 0.2) (layer F.Cu) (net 1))
 (segment (start 105.8814 91.5963) (end 107.1372 91.5963) (width 0.15) (layer F.Cu) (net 1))
 (segment (start 103.1621 90.509) (end 104.4687 90.509) (width 0.2) (layer F.Cu) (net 1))
 (segment (start 104.4687 90.509) (end 104.4814 90.4963) (width 0.2) (layer F.Cu) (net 1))
 (segment (start 101.4095 90.509) (end 102.2858 90.509) (width 0.2) (layer F.Cu) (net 1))
 (segment (start 102.2858 90.509) (end 103.1621 90.509) (width 0.2) (layer F.Cu) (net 1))
 (segment (start 99 94.6) (end 99 94.2756) (width 0.2) (layer F.Cu) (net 1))
 (segment (start 98.7432 94.0188) (end 98.7432 92.4179) (width 0.2) (layer F.Cu) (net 1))
 (segment (start 99 94.2756) (end 98.7432 94.0188) (width 0.2) (layer F.Cu) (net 1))
 (segment (start 103.25 95.85) (end 103.5589 95.85) (width 0.2) (layer F.Cu) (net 1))
 (segment (start 104.6822 95.9739) (end 105.1052 95.5509) (width 0.2) (layer F.Cu) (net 1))
 (segment (start 103.6828 95.9739) (end 104.6822 95.9739) (width 0.2) (layer F.Cu) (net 1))
 (segment (start 103.5589 95.85) (end 103.6828 95.9739) (width 0.2) (layer F.Cu) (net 1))
 (segment (start 113.6777 95.5636) (end 113.6777 95.1992) (width 0.1) (layer F.Cu) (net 1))
 (segment (start 112.9665 94.488) (end 106.6966 94.488) (width 0.1) (layer F.Cu) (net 1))
 (segment (start 113.6777 95.1992) (end 112.9665 94.488) (width 0.1) (layer F.Cu) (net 1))
 (segment (start 106.6966 94.488) (end 106.6966 93.4085) (width 0.1) (layer F.Cu) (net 1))
 (segment (start 105.1052 95.5509) (end 106.5315 95.5509) (width 0.1) (layer F.Cu) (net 1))
 (segment (start 106.6966 95.3858) (end 106.6966 94.488) (width 0.1) (layer F.Cu) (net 1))
 (segment (start 106.5315 95.5509) (end 106.6966 95.3858) (width 0.1) (layer F.Cu) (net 1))
 (segment (start 108.8771 95.5763) (end 108.8771 95.3262) (width 0.1) (layer F.Cu) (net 1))
 (segment (start 108.8771 95.3262) (end 108.0389 94.488) (width 0.1) (layer F.Cu) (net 1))
 (segment (start 108.0389 94.488) (end 106.6966 94.488) (width 0.1) (layer F.Cu) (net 1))
 (segment (start 107.1372 90.4963) (end 105.8814 90.4963) (width 0.15) (layer F.Cu) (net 2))
 (segment (start 103.75 94.6) (end 103.75 94.4462) (width 0.15) (layer F.Cu) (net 2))
 (segment (start 105.2068 91.1709) (end 105.8814 90.4963) (width 0.15) (layer F.Cu) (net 2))
 (segment (start 105.2068 92.1766) (end 105.2068 91.1709) (width 0.15) (layer F.Cu) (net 2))
 (segment (start 104.9274 92.456) (end 105.2068 92.1766) (width 0.15) (layer F.Cu) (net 2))
 (segment (start 104.9274 93.2688) (end 104.9274 92.456) (width 0.15) (layer F.Cu) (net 2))
 (segment (start 103.75 94.4462) (end 104.9274 93.2688) (width 0.15) (layer F.Cu) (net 2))
 (segment (start 103.25 94.1) (end 103.7152 94.1) (width 0.15) (layer F.Cu) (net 3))
 (segment (start 104.4814 93.3338) (end 104.4814 91.5963) (width 0.15) (layer F.Cu) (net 3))
 (segment (start 103.7152 94.1) (end 104.4814 93.3338) (width 0.15) (layer F.Cu) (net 3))
 (segment (start 103.1621 91.609) (end 104.4687 91.609) (width 0.2) (layer F.Cu) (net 3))
 (segment (start 104.4687 91.609) (end 104.4814 91.5963) (width 0.2) (layer F.Cu) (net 3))
 (segment (start 103.25 96.35) (end 103.4337 96.35) (width 0.2) (layer F.Cu) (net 16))
 (segment (start 104.3725 96.6509) (end 105.1052 96.6509) (width 0.2) (layer F.Cu) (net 16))
 (segment (start 104.013 96.2914) (end 104.3725 96.6509) (width 0.2) (layer F.Cu) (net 16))
 (segment (start 103.4923 96.2914) (end 104.013 96.2914) (width 0.2) (layer F.Cu) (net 16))
 (segment (start 103.4337 96.35) (end 103.4923 96.2914) (width 0.2) (layer F.Cu) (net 16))
 (segment (start 106.2348 96.6724) (end 105.1267 96.6724) (width 0.2) (layer F.Cu) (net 16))
 (segment (start 105.1267 96.6724) (end 105.1052 96.6509) (width 0.2) (layer F.Cu) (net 16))
 (segment (start 106.2133 96.6509) (end 106.2348 96.6724) (width 0.1) (layer F.Cu) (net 16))
 (segment (start 110.05566 96.6724) (end 108.881 96.6724) (width 0.1) (layer F.Cu) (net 21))
 (segment (start 108.881 96.6724) (end 108.8771 96.6763) (width 0.1) (layer F.Cu) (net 21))
 (segment (start 107.7348 96.6724) (end 108.8732 96.6724) (width 0.1) (layer F.Cu) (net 21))
 (segment (start 108.8732 96.6724) (end 108.8771 96.6763) (width 0.1) (layer F.Cu) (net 21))
 (segment (start 94.6443 94.9706) (end 97.1206 94.9706) (width 0.2) (layer F.Cu) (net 19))
 (segment (start 97.1206 94.9706) (end 97.25 95.1) (width 0.2) (layer F.Cu) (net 19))
 (segment (start 102.75 94.1) (end 102.75 92.8896) (width 0.2) (layer F.Cu) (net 7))
 (segment (start 102.75 92.8896) (end 102.7518 92.8878) (width 0.2) (layer F.Cu) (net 7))
 (segment (start 94.8316 93.7641) (end 96.4141 93.7641) (width 0.2) (layer F.Cu) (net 7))
 (segment (start 96.4141 93.7641) (end 97.25 94.6) (width 0.2) (layer F.Cu) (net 7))
 (segment (start 103.25 100.6) (end 103.25 102.0904) (width 0.2) (layer F.Cu) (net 7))
 (segment (start 103.25 102.0904) (end 103.251 102.0914) (width 0.2) (layer F.Cu) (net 7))
 (segment (start 100.7491 102.1041) (end 97.8567 102.1041) (width 0.2) (layer F.Cu) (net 7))
 (segment (start 97.8567 102.1041) (end 97.7519 102.2089) (width 0.2) (layer F.Cu) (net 7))
 (segment (start 100.75 100.6) (end 100.75 102.1032) (width 0.2) (layer F.Cu) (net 7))
 (segment (start 100.75 102.1032) (end 100.7491 102.1041) (width 0.2) (layer F.Cu) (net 7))
 (segment (start 97.75 100.6) (end 97.75 102.207) (width 0.2) (layer F.Cu) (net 7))
 (segment (start 97.75 102.207) (end 97.7519 102.2089) (width 0.2) (layer F.Cu) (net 7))
 (segment (start 97.25 99.1) (end 95.2862 99.1) (width 0.2) (layer F.Cu) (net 7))
 (segment (start 91.6305 100.8126) (end 91.6305 101.3072) (width 0.2) (layer F.Cu) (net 7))
 (segment (start 92.1766 100.2665) (end 91.6305 100.8126) (width 0.2) (layer F.Cu) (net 7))
 (segment (start 92.9259 100.2665) (end 92.1766 100.2665) (width 0.2) (layer F.Cu) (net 7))
 (segment (start 93.853 99.3394) (end 92.9259 100.2665) (width 0.2) (layer F.Cu) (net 7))
 (segment (start 95.0468 99.3394) (end 93.853 99.3394) (width 0.2) (layer F.Cu) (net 7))
 (segment (start 95.2862 99.1) (end 95.0468 99.3394) (width 0.2) (layer F.Cu) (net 7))
 (segment (start 100.6443 102.2089) (end 100.7491 102.1041) (width 0.1) (layer F.Cu) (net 7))
 (segment (start 97.7519 100.6019) (end 97.75 100.6) (width 0.1) (layer F.Cu) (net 7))
 (segment (start 100.7491 100.6009) (end 100.75 100.6) (width 0.1) (layer F.Cu) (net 7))
 (segment (start 103.251 100.601) (end 103.25 100.6) (width 0.1) (layer F.Cu) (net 7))
 (segment (start 102.7518 94.0982) (end 102.75 94.1) (width 0.1) (layer F.Cu) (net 7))
 (segment (start 103.75 95.6) (end 103.75 95.513) (width 0.1) (layer F.Cu) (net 18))
 (segment (start 103.75 95.513) (end 104.775 94.488) (width 0.1) (layer F.Cu) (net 18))
 (segment (start 104.775 94.488) (end 105.5966 94.488) (width 0.1) (layer F.Cu) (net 18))
 (segment (start 103.25 95.35) (end 103.5828 95.35) (width 0.15) (layer F.Cu) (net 17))
 (segment (start 103.5828 95.35) (end 105.5243 93.4085) (width 0.15) (layer F.Cu) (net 17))
 (segment (start 105.5243 93.4085) (end 105.5966 93.4085) (width 0.15) (layer F.Cu) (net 17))
 (segment (start 101.75 94.1) (end 101.75 93.4315) (width 0.2) (layer F.Cu) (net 6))
 (segment (start 101.4095 93.091) (end 101.4095 91.609) (width 0.2) (layer F.Cu) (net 6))
 (segment (start 101.75 93.4315) (end 101.4095 93.091) (width 0.2) (layer F.Cu) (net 6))
 (segment (start 98.5 94.6) (end 98.5 94.4614) (width 0.2) (layer F.Cu) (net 8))
 (segment (start 97.2432 93.2046) (end 97.2432 92.4179) (width 0.2) (layer F.Cu) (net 8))
 (segment (start 98.5 94.4614) (end 97.2432 93.2046) (width 0.2) (layer F.Cu) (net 8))
 (segment (start 97.2432 92.4179) (end 97.2432 89.9407) (width 0.2) (layer F.Cu) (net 8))
 (segment (start 96.901 89.5985) (end 96.5763 89.5985) (width 0.2) (layer F.Cu) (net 8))
 (segment (start 97.2432 89.9407) (end 96.901 89.5985) (width 0.2) (layer F.Cu) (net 8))
 (segment (start 97.75 95.35) (end 97.3979 95.35) (width 0.15) (layer F.Cu) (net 11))
 (segment (start 90.043 96.0374) (end 90.043 96.5542) (width 0.15) (layer F.Cu) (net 11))
 (segment (start 90.3859 95.6945) (end 90.043 96.0374) (width 0.15) (layer F.Cu) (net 11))
 (segment (start 94.9706 95.6945) (end 90.3859 95.6945) (width 0.15) (layer F.Cu) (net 11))
 (segment (start 95.2754 95.3897) (end 94.9706 95.6945) (width 0.15) (layer F.Cu) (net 11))
 (segment (start 97.3582 95.3897) (end 95.2754 95.3897) (width 0.15) (layer F.Cu) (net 11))
 (segment (start 97.3979 95.35) (end 97.3582 95.3897) (width 0.15) (layer F.Cu) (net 11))
 (segment (start 97.75 95.35) (end 97.7281 95.35) (width 0.1) (layer F.Cu) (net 11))
 (segment (start 90.043 97.6542) (end 90.8338 97.6542) (width 0.1) (layer F.Cu) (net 5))
 (segment (start 90.8338 97.6542) (end 91.3584 97.1296) (width 0.1) (layer F.Cu) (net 5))
 (segment (start 97.75 95.85) (end 97.5137 95.85) (width 0.15) (layer F.Cu) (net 10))
 (segment (start 94.2467 98.8949) (end 93.1838 98.8949) (width 0.15) (layer F.Cu) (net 10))
 (segment (start 94.8055 98.3361) (end 94.2467 98.8949) (width 0.15) (layer F.Cu) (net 10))
 (segment (start 94.8055 96.4946) (end 94.8055 98.3361) (width 0.15) (layer F.Cu) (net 10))
 (segment (start 95.6183 95.6818) (end 94.8055 96.4946) (width 0.15) (layer F.Cu) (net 10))
 (segment (start 97.3455 95.6818) (end 95.6183 95.6818) (width 0.15) (layer F.Cu) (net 10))
 (segment (start 97.5137 95.85) (end 97.3455 95.6818) (width 0.15) (layer F.Cu) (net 10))
 (segment (start 97.75 95.85) (end 97.7042 95.85) (width 0.1) (layer F.Cu) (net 10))
 (segment (start 92.0838 98.8949) (end 92.0838 98.4543) (width 0.15) (layer F.Cu) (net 4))
 (segment (start 92.0838 98.4543) (end 93.4085 97.1296) (width 0.15) (layer F.Cu) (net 4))
 (segment (start 93.4085 97.1296) (end 93.8584 97.1296) (width 0.15) (layer F.Cu) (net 4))
 (segment (start 92.0838 98.8949) (end 92.0931 98.8949) (width 0.1) (layer F.Cu) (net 4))
 (segment (start 97.75 99.35) (end 97.41745 99.35) (width 0.2) (layer F.Cu) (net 12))
 (segment (start 97.41745 99.35) (end 97.17405 99.5934) (width 0.2) (layer F.Cu) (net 12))
 (segment (start 93.0148 100.8761) (end 93.0148 101.3199) (width 0.2) (layer F.Cu) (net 12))
 (segment (start 97.17405 99.5934) (end 95.2627 99.5934) (width 0.2) (layer F.Cu) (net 12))
 (segment (start 95.2627 99.5934) (end 94.5388 100.3173) (width 0.2) (layer F.Cu) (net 12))
 (segment (start 94.5388 100.3173) (end 93.5736 100.3173) (width 0.2) (layer F.Cu) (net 12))
 (segment (start 93.5736 100.3173) (end 93.0148 100.8761) (width 0.2) (layer F.Cu) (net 12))
 (segment (start 93.0148 101.3199) (end 93.0148 100.9523) (width 0.1) (layer F.Cu) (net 12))
 (segment (start 95.6818 90.9567) (end 95.6818 89.604) (width 0.2) (layer F.Cu) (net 22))
 (segment (start 95.6818 89.604) (end 95.6763 89.5985) (width 0.2) (layer F.Cu) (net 22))
 (segment (start 98 94.6) (end 97.8251 94.6) (width 0.2) (layer F.Cu) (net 9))
 (segment (start 97.8251 94.6) (end 95.6818 92.4567) (width 0.2) (layer F.Cu) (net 9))
 (segment (start 96.0127 92.4567) (end 95.6818 92.4567) (width 0.15) (layer F.Cu) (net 9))
 (segment (start 97.75 99.85) (end 97.332244 99.85) (width 0.2) (layer F.Cu) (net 13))
 (segment (start 95.8208 99.949) (end 94.5388 101.231) (width 0.2) (layer F.Cu) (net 13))
 (segment (start 97.233244 99.949) (end 95.8208 99.949) (width 0.2) (layer F.Cu) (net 13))
 (segment (start 97.332244 99.85) (end 97.233244 99.949) (width 0.2) (layer F.Cu) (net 13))
 (segment (start 103.75 97.6) (end 103.8826 97.6) (width 0.2) (layer F.Cu) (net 15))
 (segment (start 103.8826 97.6) (end 105.2283 98.9457) (width 0.2) (layer F.Cu) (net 15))
 (segment (start 98.5 100.1) (end 98.0454 100.1) (width 0.2) (layer F.Cu) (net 14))
 (segment (start 96.3295 101.2825) (end 96.3295 102.2597) (width 0.2) (layer F.Cu) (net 14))
 (segment (start 97.3582 100.2538) (end 96.3295 101.2825) (width 0.2) (layer F.Cu) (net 14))
 (segment (start 97.8916 100.2538) (end 97.3582 100.2538) (width 0.2) (layer F.Cu) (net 14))
 (segment (start 98.0454 100.1) (end 97.8916 100.2538) (width 0.2) (layer F.Cu) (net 14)))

